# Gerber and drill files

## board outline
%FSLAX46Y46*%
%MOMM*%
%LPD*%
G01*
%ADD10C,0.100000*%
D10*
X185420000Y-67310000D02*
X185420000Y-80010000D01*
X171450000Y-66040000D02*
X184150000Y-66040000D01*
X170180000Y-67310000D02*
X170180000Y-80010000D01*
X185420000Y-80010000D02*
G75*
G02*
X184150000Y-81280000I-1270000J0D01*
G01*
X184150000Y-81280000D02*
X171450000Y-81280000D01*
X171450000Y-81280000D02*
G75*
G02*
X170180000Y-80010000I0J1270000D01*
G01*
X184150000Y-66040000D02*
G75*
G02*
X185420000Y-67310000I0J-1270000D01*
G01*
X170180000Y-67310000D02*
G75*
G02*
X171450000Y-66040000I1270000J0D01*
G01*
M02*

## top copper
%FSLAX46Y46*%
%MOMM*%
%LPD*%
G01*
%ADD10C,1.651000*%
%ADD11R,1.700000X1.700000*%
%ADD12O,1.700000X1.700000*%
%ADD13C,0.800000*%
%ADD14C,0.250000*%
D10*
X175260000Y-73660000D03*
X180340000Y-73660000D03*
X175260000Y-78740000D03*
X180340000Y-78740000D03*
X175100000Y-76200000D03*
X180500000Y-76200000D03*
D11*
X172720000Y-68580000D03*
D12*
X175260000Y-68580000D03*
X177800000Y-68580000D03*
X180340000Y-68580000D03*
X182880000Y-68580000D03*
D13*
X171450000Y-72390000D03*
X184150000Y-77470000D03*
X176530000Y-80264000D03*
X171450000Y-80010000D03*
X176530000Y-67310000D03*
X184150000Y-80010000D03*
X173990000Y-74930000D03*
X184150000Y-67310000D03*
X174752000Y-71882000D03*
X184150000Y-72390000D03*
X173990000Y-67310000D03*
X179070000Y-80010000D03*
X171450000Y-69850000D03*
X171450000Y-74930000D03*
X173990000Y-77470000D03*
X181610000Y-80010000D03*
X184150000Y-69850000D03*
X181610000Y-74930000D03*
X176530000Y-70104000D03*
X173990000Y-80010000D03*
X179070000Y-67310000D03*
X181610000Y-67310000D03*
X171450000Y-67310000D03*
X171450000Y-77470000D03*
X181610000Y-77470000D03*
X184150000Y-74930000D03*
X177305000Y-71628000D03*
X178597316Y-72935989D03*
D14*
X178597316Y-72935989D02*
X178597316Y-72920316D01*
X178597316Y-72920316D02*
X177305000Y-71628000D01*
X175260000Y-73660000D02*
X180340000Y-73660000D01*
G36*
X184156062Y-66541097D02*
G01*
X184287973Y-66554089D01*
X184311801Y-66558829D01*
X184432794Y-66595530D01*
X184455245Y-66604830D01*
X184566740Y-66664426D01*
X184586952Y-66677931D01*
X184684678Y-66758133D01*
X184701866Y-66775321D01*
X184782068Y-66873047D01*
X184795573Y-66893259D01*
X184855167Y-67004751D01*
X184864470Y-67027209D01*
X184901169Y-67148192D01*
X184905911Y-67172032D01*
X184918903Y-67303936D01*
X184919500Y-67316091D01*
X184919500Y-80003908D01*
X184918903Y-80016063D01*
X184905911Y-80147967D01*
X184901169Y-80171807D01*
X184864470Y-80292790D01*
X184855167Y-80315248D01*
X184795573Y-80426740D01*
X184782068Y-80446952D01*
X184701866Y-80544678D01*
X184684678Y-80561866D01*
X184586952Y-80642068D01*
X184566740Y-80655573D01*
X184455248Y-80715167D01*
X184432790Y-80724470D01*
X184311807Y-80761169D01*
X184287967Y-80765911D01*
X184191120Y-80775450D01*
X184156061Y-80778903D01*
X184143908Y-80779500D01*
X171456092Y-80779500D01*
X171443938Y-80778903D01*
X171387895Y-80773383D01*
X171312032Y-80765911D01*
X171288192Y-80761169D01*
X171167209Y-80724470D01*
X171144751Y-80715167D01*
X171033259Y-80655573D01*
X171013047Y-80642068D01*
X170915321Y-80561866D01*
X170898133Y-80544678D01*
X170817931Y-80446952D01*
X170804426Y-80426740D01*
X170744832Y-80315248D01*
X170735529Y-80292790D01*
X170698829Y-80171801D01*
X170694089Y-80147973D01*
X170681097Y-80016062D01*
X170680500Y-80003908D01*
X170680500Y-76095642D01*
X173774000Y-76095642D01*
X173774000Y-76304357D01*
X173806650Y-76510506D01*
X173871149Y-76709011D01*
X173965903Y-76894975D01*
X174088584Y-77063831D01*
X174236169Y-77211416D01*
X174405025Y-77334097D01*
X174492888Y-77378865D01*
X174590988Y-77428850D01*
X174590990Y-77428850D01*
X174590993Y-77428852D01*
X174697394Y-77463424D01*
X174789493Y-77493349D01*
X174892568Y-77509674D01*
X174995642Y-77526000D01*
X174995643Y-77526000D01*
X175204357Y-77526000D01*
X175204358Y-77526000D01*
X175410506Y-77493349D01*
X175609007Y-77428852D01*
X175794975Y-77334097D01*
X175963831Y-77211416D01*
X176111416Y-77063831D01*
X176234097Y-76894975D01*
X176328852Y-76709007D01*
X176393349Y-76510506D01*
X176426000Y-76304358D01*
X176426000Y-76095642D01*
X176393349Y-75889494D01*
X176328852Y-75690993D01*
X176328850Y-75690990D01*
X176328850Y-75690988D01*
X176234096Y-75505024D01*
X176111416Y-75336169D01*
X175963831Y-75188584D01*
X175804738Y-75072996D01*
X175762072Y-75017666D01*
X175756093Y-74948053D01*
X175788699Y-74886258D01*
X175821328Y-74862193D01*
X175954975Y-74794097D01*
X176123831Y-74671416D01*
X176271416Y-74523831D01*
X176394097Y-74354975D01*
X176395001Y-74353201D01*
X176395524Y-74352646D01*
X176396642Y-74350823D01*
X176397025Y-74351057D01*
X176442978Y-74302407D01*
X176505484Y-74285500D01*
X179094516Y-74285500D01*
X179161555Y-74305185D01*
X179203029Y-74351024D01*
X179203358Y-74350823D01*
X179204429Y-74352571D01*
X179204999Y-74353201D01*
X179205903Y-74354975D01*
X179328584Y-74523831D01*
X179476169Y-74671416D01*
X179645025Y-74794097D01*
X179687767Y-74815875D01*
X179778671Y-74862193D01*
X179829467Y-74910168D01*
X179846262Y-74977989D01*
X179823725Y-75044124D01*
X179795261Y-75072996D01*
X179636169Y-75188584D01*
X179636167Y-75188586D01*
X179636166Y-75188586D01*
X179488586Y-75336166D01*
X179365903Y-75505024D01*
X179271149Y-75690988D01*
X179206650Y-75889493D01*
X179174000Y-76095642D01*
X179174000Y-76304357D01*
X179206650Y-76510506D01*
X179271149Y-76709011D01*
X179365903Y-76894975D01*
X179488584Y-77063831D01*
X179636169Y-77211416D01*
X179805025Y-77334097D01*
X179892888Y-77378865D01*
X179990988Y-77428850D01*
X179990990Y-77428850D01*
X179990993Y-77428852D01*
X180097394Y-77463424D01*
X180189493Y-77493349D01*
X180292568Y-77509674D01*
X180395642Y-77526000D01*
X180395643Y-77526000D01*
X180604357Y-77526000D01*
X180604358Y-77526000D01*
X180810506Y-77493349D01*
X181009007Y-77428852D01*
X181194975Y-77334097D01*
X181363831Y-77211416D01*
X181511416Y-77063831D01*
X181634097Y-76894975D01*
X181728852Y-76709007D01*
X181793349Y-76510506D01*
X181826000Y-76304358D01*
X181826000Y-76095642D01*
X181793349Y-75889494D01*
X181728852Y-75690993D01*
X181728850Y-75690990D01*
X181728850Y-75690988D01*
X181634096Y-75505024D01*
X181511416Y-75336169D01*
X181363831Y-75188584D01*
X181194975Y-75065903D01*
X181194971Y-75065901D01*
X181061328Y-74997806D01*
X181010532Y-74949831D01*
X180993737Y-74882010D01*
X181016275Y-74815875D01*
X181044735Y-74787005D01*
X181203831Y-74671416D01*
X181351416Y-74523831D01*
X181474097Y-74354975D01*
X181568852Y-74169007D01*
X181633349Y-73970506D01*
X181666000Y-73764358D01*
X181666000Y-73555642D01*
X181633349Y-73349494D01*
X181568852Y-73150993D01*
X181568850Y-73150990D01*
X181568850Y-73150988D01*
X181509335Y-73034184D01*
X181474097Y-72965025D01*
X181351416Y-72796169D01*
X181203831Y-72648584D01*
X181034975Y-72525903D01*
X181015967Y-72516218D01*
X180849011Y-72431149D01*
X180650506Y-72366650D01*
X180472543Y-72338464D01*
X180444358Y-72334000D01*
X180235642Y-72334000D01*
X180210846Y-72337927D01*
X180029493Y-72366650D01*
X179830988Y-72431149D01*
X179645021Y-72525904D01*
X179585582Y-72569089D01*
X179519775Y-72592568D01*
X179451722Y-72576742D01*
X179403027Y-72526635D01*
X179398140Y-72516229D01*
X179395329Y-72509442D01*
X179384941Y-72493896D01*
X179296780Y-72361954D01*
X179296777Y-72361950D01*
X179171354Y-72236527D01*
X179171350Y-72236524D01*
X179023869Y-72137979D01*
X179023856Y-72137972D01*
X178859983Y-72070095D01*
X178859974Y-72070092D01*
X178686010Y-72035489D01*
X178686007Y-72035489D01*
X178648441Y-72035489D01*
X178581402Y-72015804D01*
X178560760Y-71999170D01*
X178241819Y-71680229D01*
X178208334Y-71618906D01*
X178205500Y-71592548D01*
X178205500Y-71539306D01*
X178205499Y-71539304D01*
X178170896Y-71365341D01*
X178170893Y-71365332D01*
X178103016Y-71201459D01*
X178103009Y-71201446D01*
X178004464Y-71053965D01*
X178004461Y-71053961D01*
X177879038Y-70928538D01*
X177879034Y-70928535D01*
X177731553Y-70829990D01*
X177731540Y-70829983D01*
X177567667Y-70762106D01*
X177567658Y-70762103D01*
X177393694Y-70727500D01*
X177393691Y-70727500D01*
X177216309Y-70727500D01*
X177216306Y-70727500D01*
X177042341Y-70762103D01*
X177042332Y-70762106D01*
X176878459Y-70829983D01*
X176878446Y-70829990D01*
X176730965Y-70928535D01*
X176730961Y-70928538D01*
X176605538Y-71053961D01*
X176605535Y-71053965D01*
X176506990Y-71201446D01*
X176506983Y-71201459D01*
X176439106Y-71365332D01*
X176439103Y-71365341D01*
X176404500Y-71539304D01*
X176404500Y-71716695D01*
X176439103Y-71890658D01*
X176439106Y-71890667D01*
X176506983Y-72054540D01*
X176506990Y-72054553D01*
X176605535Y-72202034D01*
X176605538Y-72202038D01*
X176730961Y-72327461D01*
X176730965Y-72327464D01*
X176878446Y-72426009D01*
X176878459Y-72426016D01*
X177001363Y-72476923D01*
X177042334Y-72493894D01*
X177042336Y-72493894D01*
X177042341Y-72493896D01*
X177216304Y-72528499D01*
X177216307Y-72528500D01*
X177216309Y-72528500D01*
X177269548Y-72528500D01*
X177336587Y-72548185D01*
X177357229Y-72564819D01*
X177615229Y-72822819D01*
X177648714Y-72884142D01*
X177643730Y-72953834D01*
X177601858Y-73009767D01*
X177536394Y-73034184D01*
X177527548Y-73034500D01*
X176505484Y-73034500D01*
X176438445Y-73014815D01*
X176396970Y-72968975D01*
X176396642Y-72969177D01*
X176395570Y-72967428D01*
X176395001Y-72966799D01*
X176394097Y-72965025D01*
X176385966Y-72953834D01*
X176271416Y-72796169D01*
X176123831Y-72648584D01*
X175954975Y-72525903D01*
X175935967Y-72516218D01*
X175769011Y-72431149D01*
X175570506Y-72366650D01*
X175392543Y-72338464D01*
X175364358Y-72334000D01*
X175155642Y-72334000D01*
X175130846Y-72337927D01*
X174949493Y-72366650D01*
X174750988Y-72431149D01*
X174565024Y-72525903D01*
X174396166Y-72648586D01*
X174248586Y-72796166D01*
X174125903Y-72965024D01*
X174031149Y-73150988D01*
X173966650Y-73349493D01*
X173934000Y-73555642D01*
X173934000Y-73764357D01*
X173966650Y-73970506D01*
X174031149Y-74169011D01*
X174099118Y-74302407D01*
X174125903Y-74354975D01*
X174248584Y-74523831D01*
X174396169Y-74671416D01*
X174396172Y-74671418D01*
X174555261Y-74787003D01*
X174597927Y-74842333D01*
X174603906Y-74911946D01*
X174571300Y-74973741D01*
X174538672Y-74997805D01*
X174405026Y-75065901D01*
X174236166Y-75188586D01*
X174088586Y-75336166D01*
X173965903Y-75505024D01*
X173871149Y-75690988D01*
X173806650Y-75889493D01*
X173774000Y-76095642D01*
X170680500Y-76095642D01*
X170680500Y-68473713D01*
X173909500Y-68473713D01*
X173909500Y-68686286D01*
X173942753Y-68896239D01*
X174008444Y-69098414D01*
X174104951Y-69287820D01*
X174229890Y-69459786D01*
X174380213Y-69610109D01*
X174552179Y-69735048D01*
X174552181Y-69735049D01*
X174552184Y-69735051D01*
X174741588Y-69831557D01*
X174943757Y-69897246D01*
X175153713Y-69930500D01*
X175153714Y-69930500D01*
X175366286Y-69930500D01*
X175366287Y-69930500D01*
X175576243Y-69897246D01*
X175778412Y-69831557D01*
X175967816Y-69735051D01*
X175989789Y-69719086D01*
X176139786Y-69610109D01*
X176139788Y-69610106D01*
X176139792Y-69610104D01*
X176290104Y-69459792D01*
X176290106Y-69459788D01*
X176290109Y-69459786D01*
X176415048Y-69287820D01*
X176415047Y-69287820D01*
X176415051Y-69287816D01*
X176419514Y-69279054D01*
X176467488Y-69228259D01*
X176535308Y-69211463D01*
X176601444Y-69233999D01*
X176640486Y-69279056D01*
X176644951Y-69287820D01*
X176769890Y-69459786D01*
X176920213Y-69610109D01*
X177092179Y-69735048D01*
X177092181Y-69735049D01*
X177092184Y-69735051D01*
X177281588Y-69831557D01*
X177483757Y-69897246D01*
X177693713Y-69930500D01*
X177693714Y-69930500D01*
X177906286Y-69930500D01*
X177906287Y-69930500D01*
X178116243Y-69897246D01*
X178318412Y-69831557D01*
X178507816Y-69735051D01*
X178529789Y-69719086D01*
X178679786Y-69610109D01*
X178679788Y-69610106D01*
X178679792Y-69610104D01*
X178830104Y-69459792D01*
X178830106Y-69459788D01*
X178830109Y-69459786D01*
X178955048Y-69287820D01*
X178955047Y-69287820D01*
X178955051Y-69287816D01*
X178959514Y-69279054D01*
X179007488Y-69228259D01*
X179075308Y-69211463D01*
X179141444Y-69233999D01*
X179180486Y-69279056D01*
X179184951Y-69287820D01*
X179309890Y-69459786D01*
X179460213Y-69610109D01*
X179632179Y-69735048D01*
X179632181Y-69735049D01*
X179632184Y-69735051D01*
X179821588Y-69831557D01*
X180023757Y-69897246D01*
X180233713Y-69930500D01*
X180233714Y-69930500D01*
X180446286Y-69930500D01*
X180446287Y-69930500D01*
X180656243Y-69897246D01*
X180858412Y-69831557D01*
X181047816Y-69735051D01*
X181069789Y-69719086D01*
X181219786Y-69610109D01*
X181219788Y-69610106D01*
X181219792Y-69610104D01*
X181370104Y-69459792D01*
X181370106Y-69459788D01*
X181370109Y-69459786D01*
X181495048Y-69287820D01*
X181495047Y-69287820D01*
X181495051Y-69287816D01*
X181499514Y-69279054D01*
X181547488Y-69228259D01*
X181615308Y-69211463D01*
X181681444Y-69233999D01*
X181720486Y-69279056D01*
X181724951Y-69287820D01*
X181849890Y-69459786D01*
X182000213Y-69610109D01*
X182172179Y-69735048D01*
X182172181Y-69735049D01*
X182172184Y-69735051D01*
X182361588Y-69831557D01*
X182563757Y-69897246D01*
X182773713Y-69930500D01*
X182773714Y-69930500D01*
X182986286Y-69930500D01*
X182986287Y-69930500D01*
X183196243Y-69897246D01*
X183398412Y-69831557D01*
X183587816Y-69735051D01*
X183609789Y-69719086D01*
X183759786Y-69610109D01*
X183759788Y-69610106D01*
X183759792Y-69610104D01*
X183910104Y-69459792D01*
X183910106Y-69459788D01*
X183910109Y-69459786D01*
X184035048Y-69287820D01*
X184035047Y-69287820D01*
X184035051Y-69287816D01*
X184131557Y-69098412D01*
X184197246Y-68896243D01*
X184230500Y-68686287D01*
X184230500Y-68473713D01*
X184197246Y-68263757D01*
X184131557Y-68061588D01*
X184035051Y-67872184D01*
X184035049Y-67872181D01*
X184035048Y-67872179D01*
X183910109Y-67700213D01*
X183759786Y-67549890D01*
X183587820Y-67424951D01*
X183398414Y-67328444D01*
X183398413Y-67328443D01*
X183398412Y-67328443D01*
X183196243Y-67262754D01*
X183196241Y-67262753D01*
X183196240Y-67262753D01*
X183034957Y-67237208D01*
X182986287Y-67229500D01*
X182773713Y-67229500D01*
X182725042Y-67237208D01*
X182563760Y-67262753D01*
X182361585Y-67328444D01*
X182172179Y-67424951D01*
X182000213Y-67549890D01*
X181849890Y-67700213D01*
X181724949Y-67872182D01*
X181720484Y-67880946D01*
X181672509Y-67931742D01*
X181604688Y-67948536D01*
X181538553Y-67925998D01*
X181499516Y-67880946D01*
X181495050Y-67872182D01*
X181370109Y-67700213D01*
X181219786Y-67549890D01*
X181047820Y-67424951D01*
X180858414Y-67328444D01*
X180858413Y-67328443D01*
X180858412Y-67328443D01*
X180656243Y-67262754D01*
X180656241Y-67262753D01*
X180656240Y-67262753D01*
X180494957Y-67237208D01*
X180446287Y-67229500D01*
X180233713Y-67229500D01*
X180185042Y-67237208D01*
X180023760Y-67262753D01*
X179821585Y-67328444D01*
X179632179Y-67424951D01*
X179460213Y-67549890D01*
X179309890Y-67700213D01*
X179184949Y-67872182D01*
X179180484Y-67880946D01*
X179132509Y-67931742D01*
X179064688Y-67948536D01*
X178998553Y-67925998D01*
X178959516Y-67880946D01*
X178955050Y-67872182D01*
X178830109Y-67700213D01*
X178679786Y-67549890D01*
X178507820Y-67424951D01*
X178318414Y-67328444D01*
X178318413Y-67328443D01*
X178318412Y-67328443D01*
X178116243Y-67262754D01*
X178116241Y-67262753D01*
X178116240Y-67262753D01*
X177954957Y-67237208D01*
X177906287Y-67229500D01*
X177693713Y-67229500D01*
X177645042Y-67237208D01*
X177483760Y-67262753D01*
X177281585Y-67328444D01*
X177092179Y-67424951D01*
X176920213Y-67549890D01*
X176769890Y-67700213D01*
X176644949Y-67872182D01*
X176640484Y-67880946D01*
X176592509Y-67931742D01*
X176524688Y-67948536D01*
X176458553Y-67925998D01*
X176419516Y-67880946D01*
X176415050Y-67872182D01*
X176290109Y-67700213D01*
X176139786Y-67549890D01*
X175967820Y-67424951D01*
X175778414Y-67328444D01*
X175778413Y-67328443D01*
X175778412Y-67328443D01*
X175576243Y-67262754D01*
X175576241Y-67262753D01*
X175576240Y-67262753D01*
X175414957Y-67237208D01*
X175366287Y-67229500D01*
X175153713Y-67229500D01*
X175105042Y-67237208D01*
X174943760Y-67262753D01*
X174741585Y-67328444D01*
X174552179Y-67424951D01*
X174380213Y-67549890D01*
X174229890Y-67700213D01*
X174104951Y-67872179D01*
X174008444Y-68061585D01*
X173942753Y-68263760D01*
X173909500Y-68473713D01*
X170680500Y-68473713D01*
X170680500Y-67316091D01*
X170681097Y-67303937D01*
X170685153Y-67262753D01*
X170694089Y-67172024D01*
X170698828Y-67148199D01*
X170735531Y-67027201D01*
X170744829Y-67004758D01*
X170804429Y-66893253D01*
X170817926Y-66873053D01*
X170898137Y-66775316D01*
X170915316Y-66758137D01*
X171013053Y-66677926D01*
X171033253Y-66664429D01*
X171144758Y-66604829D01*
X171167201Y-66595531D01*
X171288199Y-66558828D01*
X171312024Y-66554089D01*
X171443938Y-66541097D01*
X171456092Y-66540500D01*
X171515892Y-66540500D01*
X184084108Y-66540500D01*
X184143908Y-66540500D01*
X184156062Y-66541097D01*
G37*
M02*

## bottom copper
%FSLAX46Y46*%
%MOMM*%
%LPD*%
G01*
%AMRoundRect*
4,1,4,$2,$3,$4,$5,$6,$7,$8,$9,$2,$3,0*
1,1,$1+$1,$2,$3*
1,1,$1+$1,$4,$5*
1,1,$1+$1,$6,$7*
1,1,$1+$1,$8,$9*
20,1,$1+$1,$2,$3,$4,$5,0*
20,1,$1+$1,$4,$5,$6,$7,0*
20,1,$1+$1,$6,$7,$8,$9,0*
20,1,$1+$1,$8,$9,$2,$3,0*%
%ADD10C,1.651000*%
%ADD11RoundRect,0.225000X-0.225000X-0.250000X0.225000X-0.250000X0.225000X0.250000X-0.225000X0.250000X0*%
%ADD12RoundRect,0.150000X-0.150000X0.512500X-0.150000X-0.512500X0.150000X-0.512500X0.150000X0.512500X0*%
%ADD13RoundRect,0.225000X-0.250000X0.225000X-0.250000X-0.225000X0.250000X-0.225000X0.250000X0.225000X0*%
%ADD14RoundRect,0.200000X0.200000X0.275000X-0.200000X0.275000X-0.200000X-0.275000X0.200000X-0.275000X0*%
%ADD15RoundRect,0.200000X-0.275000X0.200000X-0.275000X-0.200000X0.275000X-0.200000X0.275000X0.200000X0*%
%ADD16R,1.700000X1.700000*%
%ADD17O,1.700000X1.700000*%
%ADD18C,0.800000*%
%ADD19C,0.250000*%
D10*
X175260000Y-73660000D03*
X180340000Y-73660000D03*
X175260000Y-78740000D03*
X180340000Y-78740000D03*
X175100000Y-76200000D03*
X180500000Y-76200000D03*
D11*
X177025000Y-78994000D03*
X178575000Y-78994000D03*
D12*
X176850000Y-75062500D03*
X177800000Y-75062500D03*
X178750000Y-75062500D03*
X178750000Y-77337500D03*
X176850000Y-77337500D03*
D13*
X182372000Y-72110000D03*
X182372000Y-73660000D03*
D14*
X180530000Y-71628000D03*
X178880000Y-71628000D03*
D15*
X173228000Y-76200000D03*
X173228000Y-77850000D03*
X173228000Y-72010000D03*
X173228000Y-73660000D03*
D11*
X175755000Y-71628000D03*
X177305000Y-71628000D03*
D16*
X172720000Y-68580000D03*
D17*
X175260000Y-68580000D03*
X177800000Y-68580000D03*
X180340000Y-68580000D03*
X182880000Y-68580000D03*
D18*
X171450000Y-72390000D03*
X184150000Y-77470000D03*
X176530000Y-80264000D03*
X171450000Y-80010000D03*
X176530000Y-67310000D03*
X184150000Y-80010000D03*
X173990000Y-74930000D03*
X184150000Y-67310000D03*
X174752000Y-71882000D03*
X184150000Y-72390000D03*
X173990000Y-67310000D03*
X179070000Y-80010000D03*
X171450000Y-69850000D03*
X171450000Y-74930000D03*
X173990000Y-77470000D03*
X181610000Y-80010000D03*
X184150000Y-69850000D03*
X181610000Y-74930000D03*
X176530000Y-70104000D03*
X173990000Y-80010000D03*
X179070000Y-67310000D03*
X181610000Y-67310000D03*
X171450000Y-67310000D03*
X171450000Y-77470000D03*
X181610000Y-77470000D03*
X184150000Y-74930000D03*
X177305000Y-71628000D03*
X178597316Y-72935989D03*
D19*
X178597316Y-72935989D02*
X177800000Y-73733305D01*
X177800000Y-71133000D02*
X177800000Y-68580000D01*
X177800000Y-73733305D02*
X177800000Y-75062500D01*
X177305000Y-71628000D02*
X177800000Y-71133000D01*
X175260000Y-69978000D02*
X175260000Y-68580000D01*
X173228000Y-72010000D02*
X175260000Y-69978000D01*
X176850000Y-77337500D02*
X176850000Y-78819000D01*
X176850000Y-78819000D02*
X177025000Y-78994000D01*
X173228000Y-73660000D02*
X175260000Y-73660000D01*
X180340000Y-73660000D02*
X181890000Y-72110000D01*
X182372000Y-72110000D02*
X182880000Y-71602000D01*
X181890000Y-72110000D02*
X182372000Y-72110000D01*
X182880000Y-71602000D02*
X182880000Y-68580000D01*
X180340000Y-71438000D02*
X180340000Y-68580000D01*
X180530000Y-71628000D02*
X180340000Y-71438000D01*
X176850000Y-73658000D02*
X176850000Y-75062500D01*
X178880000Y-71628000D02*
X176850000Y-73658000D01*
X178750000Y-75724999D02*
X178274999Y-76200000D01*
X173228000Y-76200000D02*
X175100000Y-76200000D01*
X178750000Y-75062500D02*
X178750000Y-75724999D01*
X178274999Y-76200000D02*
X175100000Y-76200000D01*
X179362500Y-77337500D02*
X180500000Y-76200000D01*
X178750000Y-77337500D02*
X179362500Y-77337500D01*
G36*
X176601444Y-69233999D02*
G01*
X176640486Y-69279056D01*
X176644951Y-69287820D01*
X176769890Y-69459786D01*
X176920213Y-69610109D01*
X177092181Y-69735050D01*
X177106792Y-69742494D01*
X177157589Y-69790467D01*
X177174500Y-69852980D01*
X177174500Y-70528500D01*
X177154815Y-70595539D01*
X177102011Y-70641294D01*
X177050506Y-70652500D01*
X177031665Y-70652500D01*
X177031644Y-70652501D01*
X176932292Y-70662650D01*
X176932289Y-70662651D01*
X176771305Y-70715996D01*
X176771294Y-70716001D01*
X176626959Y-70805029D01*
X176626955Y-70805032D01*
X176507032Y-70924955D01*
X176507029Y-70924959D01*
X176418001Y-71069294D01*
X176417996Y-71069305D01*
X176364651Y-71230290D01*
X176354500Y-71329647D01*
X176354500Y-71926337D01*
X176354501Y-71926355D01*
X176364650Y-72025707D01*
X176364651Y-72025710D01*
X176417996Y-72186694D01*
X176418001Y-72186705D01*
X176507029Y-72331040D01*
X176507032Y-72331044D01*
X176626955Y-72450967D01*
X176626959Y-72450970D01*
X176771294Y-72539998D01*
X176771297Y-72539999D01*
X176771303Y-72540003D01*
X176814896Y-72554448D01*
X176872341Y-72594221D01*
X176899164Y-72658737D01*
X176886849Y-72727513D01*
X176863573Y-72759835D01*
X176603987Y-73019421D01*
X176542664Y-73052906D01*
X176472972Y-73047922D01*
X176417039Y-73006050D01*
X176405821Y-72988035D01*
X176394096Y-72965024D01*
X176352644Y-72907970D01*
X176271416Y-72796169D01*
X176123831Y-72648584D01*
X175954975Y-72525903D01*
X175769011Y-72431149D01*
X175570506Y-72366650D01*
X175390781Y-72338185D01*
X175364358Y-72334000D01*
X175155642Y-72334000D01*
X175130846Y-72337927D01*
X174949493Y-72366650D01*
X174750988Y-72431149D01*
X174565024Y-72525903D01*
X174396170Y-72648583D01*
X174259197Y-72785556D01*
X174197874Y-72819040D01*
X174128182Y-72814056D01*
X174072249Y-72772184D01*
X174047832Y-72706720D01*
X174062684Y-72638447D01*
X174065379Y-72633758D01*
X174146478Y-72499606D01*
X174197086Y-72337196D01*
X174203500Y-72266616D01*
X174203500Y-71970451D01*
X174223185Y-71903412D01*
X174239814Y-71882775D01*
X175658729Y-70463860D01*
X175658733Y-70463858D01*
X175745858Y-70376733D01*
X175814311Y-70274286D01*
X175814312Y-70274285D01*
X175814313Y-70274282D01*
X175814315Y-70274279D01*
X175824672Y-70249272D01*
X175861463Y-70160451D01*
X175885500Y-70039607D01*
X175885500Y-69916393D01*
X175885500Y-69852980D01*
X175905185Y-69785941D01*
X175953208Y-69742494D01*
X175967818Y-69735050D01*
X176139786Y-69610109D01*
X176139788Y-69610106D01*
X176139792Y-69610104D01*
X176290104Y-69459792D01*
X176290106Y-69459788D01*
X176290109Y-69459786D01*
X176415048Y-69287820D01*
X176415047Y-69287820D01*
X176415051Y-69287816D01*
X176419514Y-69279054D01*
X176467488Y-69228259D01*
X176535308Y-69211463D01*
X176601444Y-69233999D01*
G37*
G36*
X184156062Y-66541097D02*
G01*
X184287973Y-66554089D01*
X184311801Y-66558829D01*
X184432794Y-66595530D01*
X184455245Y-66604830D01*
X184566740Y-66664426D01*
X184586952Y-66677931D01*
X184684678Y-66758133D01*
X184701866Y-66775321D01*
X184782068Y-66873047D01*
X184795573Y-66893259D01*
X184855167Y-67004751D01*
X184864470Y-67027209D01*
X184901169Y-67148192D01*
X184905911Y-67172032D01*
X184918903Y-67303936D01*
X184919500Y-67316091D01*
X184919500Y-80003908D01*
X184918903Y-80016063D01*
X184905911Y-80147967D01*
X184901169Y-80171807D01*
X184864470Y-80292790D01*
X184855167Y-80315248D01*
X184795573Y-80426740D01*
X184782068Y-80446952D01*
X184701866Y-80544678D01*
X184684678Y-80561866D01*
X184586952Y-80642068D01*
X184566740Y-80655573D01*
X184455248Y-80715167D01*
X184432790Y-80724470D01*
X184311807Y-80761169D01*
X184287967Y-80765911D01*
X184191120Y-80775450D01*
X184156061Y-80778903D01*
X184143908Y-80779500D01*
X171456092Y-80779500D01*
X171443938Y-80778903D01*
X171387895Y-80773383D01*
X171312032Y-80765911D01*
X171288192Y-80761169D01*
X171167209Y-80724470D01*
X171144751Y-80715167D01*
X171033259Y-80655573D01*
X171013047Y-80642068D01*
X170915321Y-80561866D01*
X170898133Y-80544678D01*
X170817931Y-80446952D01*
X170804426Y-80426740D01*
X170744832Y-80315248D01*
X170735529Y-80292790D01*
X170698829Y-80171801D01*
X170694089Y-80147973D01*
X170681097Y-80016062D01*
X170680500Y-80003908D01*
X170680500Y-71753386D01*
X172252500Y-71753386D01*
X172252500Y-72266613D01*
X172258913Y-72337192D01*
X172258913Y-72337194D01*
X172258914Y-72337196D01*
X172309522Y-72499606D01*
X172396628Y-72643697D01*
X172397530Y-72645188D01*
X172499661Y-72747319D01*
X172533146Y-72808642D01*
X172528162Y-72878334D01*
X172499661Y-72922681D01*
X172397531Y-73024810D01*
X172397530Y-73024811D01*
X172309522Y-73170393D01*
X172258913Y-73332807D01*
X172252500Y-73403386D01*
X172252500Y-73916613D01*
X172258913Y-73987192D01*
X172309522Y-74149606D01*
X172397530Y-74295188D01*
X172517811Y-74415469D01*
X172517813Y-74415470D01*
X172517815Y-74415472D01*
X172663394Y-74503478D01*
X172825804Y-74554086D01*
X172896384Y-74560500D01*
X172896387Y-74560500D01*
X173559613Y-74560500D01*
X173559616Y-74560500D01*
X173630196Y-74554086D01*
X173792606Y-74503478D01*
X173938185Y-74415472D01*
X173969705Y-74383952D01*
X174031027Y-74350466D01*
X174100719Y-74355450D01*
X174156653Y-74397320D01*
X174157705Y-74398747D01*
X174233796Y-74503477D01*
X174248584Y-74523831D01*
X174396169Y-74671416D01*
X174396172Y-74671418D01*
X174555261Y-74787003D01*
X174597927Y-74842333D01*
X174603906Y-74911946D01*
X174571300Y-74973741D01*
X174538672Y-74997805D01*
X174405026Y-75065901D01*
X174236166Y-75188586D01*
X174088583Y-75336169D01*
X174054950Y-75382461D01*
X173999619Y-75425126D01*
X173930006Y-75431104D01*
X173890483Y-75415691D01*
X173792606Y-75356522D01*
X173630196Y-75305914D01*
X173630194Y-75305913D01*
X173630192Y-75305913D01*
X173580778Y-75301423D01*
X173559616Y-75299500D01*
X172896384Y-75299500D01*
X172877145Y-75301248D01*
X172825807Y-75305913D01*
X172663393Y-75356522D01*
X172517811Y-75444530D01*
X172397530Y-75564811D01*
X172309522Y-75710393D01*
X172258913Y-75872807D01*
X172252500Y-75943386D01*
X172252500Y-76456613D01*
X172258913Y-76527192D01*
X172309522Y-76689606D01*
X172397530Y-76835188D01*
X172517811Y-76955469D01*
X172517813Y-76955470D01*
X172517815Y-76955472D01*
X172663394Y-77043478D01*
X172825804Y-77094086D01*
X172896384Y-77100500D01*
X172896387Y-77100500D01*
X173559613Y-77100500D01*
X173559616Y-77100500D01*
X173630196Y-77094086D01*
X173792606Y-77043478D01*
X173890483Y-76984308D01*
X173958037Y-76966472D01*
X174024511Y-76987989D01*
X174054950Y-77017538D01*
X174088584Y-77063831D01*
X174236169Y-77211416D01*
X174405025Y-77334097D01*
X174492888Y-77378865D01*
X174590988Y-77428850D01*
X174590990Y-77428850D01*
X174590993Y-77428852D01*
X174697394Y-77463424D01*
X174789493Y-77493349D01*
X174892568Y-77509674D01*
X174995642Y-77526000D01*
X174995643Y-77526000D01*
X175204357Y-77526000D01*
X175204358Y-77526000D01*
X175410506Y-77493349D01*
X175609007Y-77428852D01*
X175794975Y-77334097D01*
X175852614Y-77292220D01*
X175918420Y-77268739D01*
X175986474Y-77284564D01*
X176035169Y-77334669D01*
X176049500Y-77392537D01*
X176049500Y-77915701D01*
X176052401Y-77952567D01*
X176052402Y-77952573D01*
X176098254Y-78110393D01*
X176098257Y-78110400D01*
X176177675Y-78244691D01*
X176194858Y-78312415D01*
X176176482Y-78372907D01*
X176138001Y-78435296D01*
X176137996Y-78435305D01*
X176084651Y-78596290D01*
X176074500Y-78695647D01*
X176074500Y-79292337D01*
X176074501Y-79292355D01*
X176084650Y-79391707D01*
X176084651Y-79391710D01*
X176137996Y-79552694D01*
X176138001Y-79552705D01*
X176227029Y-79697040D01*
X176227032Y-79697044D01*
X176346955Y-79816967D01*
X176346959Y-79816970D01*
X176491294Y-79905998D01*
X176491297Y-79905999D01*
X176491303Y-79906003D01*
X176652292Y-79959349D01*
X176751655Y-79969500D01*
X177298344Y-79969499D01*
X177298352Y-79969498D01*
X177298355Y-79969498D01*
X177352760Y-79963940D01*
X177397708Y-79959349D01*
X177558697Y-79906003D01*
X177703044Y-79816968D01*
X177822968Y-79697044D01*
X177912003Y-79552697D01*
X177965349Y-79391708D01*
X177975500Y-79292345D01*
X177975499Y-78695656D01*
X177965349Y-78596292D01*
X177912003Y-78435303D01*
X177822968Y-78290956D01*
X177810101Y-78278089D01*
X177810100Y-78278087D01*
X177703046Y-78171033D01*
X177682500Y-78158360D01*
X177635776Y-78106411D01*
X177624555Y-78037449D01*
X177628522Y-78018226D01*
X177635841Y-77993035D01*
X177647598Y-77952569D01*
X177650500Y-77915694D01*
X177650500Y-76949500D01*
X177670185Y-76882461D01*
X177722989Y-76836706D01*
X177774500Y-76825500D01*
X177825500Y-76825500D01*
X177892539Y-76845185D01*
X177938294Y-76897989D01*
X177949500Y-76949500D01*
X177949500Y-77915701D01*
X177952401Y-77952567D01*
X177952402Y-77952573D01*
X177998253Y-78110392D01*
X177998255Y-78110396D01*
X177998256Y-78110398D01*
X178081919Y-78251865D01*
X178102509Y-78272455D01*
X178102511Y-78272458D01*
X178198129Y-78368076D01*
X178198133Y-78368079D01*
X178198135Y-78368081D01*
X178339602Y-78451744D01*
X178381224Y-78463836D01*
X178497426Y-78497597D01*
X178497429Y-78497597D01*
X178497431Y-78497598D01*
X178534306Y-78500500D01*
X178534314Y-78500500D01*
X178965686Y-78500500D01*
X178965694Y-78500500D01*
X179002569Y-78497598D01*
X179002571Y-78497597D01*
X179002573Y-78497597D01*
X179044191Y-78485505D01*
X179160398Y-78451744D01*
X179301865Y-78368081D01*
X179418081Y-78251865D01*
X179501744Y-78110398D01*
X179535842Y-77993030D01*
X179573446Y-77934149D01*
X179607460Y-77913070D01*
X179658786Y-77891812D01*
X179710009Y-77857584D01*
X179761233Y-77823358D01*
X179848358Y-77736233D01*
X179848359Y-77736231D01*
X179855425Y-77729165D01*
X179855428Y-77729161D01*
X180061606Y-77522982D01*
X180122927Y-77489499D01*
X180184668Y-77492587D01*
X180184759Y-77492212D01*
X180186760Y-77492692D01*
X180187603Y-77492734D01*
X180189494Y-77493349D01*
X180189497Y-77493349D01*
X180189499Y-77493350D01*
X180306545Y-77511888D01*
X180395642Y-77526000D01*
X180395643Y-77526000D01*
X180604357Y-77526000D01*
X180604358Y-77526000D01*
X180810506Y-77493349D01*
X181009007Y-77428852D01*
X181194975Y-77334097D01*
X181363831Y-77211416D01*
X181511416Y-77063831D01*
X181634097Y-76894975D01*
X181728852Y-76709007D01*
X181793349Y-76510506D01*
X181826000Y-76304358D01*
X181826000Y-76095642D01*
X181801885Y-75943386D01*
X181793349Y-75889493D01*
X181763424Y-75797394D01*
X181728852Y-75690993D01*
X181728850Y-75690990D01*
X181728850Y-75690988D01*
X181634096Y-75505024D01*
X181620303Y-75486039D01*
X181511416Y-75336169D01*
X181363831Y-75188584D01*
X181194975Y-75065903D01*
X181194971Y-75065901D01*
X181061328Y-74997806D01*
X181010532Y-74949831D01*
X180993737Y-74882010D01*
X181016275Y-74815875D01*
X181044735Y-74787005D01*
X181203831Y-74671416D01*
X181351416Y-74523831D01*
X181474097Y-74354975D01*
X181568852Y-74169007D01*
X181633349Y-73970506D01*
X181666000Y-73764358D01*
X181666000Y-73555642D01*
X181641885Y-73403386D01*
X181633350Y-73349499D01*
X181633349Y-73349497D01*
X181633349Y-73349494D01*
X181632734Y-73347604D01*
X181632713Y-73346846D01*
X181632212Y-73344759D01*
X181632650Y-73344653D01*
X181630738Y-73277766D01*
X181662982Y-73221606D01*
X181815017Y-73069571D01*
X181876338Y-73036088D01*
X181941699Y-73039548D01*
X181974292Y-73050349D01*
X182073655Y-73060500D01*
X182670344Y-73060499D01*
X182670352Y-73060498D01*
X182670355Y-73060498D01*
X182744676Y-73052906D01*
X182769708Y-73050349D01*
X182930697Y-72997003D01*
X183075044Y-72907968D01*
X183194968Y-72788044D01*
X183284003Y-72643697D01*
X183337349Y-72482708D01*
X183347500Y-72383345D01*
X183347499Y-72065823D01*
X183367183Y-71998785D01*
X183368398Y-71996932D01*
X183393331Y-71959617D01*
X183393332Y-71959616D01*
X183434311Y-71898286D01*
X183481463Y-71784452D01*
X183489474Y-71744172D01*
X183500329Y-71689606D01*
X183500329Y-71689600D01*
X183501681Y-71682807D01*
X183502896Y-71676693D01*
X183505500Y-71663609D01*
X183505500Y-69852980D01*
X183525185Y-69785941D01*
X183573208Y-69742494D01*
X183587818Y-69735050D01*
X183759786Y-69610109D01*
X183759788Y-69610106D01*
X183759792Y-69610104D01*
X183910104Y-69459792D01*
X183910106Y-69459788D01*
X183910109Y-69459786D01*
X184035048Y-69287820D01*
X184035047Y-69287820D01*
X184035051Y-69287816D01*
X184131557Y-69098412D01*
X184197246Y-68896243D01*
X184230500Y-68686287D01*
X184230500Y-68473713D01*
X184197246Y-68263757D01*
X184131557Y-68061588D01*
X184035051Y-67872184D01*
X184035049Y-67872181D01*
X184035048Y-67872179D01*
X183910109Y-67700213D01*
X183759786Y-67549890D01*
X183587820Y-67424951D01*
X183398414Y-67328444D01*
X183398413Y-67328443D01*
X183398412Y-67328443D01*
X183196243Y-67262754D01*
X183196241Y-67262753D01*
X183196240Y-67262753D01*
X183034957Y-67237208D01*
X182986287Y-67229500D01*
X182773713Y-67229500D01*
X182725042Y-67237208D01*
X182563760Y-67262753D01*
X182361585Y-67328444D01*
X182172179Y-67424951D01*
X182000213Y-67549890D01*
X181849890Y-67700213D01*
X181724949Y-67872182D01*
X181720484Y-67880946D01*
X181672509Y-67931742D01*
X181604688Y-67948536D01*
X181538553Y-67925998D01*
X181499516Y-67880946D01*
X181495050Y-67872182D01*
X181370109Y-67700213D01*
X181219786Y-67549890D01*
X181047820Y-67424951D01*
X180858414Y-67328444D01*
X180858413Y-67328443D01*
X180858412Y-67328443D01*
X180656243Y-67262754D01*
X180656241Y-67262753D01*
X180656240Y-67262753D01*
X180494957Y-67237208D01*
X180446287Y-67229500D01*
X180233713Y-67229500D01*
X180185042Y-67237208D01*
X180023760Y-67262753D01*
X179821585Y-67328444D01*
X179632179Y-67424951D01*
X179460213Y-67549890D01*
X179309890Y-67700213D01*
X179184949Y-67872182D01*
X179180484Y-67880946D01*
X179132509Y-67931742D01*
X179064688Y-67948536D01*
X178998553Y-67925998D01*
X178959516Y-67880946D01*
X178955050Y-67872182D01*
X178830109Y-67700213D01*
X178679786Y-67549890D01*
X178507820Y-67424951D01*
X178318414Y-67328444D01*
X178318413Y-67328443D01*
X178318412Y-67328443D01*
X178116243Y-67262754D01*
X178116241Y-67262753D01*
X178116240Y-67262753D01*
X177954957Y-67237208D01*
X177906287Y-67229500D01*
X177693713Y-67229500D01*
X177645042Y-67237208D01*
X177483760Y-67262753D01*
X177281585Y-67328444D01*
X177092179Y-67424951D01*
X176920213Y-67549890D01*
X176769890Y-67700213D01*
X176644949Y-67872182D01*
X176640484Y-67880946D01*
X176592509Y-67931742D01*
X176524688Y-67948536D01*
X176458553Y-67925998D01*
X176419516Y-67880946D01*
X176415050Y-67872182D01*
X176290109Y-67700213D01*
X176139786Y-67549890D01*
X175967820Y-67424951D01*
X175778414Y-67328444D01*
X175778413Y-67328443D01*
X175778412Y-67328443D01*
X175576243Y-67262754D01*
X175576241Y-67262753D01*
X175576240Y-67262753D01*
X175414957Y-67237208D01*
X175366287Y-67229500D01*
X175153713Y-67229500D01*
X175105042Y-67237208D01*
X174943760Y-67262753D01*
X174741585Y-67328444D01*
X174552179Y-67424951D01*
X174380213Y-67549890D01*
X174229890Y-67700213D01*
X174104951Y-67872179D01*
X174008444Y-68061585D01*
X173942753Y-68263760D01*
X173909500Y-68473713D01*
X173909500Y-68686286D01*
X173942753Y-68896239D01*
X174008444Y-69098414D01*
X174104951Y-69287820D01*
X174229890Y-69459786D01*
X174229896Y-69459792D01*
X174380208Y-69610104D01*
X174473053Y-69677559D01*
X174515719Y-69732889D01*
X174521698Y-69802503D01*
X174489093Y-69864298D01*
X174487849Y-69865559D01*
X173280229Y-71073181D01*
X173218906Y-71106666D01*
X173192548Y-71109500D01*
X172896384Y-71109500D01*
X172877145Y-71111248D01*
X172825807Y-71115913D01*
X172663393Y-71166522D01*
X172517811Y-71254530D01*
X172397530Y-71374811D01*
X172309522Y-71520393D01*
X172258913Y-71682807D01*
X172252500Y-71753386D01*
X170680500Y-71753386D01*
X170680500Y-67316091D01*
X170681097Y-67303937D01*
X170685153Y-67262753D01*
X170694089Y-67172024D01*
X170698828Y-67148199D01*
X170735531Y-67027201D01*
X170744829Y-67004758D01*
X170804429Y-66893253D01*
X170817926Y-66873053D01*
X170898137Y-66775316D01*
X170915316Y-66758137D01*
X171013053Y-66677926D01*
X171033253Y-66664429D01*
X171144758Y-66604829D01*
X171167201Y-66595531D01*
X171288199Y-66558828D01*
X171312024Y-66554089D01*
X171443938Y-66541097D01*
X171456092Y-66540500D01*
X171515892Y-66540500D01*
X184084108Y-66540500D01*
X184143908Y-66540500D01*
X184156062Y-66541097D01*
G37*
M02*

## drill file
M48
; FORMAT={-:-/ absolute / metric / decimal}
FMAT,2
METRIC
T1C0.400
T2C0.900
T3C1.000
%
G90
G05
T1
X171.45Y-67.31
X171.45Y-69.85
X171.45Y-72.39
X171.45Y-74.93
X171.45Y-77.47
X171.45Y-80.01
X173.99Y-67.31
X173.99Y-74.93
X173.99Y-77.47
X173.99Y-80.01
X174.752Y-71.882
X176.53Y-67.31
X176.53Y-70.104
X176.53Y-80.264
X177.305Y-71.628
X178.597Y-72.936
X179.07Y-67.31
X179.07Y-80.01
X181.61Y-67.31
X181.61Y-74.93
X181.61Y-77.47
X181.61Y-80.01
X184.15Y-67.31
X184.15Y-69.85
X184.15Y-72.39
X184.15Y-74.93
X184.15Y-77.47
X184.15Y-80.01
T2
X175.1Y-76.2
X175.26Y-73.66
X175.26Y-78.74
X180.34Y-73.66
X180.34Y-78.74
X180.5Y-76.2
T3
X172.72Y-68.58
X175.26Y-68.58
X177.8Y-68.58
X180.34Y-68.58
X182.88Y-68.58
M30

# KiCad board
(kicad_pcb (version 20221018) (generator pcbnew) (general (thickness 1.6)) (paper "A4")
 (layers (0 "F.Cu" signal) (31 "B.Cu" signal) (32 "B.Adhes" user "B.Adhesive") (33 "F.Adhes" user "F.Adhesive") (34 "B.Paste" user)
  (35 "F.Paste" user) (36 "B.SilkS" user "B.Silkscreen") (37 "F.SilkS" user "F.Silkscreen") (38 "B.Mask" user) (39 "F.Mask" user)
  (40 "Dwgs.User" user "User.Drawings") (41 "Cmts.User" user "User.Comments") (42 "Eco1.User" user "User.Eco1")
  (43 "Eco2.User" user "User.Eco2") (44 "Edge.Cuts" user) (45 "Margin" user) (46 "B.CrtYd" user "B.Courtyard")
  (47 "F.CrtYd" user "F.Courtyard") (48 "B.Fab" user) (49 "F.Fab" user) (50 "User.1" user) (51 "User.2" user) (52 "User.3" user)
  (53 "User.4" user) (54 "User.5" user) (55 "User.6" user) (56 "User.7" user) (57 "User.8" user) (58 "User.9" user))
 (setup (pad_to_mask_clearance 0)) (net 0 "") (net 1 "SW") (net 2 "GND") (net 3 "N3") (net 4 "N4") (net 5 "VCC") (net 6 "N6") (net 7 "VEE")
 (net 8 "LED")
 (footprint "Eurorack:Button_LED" (layer "F.Cu") (at 177.8 76.2)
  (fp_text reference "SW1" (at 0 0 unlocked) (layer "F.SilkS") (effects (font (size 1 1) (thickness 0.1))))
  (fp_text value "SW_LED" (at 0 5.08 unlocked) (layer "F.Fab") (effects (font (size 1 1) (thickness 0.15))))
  (pad "1" thru_hole circle (at -2.54 -2.54) (size 1.651 1.651) (drill 0.9) (layers "*.Cu" "*.Mask") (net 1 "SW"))
  (pad "1" thru_hole circle (at 2.54 -2.54) (size 1.651 1.651) (drill 0.9) (layers "*.Cu" "*.Mask") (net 1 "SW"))
  (pad "2" thru_hole circle (at -2.54 2.54) (size 1.651 1.651) (drill 0.9) (layers "*.Cu" "*.Mask") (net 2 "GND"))
  (pad "2" thru_hole circle (at 2.54 2.54) (size 1.651 1.651) (drill 0.9) (layers "*.Cu" "*.Mask") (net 2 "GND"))
  (pad "3" thru_hole circle (at -2.7 0) (size 1.651 1.651) (drill 0.9) (layers "*.Cu" "*.Mask") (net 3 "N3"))
  (pad "4" thru_hole circle (at 2.7 0) (size 1.651 1.651) (drill 0.9) (layers "*.Cu" "*.Mask") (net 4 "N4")))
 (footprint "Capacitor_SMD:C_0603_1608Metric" (layer "B.Cu") (at 177.8 78.994)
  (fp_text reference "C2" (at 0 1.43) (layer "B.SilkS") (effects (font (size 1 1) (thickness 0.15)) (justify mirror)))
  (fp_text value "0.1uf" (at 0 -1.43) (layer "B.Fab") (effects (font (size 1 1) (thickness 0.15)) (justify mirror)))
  (pad "1" smd roundrect (at -0.775 0) (size 0.9 0.95) (layers "B.Cu" "B.Paste" "B.Mask") (roundrect_rratio 0.25) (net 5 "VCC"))
  (pad "2" smd roundrect (at 0.775 0) (size 0.9 0.95) (layers "B.Cu" "B.Paste" "B.Mask") (roundrect_rratio 0.25) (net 2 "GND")))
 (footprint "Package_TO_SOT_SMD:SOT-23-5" (layer "B.Cu") (at 177.8 76.2 -90)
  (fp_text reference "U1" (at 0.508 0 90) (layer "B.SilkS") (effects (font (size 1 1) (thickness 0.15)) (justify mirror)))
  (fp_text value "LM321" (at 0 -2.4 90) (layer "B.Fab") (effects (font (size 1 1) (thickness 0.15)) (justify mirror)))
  (pad "1" smd roundrect (at -1.1375 0.95 270) (size 1.325 0.6) (layers "B.Cu" "B.Paste" "B.Mask") (roundrect_rratio 0.25) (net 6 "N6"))
  (pad "2" smd roundrect (at -1.1375 0 270) (size 1.325 0.6) (layers "B.Cu" "B.Paste" "B.Mask") (roundrect_rratio 0.25) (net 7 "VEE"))
  (pad "3" smd roundrect (at -1.1375 -0.95 270) (size 1.325 0.6) (layers "B.Cu" "B.Paste" "B.Mask") (roundrect_rratio 0.25) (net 3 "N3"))
  (pad "4" smd roundrect (at 1.1375 -0.95 270) (size 1.325 0.6) (layers "B.Cu" "B.Paste" "B.Mask") (roundrect_rratio 0.25) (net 4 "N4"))
  (pad "5" smd roundrect (at 1.1375 0.95 270) (size 1.325 0.6) (layers "B.Cu" "B.Paste" "B.Mask") (roundrect_rratio 0.25) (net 5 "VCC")))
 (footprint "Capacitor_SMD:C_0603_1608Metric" (layer "B.Cu") (at 182.372 72.885 -90)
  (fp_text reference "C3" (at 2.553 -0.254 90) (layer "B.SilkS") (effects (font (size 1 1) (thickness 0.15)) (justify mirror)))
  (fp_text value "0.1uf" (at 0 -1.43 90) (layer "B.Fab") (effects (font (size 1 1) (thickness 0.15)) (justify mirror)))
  (pad "1" smd roundrect (at -0.775 0 270) (size 0.9 0.95) (layers "B.Cu" "B.Paste" "B.Mask") (roundrect_rratio 0.25) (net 1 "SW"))
  (pad "2" smd roundrect (at 0.775 0 270) (size 0.9 0.95) (layers "B.Cu" "B.Paste" "B.Mask") (roundrect_rratio 0.25) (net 2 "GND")))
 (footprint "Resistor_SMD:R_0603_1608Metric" (layer "B.Cu") (at 179.705 71.628 180)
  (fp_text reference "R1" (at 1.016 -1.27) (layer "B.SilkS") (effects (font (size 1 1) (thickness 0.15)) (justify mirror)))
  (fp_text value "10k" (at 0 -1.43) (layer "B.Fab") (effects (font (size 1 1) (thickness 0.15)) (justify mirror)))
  (pad "1" smd roundrect (at -0.825 0 180) (size 0.8 0.95) (layers "B.Cu" "B.Paste" "B.Mask") (roundrect_rratio 0.25) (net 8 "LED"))
  (pad "2" smd roundrect (at 0.825 0 180) (size 0.8 0.95) (layers "B.Cu" "B.Paste" "B.Mask") (roundrect_rratio 0.25) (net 6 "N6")))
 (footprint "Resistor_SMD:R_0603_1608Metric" (layer "B.Cu") (at 173.228 77.025 -90)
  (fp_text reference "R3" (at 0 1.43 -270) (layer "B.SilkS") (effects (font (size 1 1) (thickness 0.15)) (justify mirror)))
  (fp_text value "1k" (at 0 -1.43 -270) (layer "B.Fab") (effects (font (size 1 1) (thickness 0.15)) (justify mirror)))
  (pad "1" smd roundrect (at -0.825 0 270) (size 0.8 0.95) (layers "B.Cu" "B.Paste" "B.Mask") (roundrect_rratio 0.25) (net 3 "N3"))
  (pad "2" smd roundrect (at 0.825 0 270) (size 0.8 0.95) (layers "B.Cu" "B.Paste" "B.Mask") (roundrect_rratio 0.25) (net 2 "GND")))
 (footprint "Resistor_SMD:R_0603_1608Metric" (layer "B.Cu") (at 173.228 72.835 -90)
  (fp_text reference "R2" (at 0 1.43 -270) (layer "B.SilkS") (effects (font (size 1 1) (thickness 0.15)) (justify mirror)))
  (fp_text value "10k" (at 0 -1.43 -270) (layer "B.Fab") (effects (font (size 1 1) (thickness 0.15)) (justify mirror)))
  (pad "1" smd roundrect (at -0.825 0 270) (size 0.8 0.95) (layers "B.Cu" "B.Paste" "B.Mask") (roundrect_rratio 0.25) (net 5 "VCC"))
  (pad "2" smd roundrect (at 0.825 0 270) (size 0.8 0.95) (layers "B.Cu" "B.Paste" "B.Mask") (roundrect_rratio 0.25) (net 1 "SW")))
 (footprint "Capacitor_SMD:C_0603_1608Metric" (layer "B.Cu") (at 176.53 71.628)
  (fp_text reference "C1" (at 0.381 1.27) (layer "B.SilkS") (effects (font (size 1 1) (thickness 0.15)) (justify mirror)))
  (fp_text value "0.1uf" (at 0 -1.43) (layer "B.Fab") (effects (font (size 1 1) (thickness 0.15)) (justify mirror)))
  (pad "1" smd roundrect (at -0.775 0) (size 0.9 0.95) (layers "B.Cu" "B.Paste" "B.Mask") (roundrect_rratio 0.25) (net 2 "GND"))
  (pad "2" smd roundrect (at 0.775 0) (size 0.9 0.95) (layers "B.Cu" "B.Paste" "B.Mask") (roundrect_rratio 0.25) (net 7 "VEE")))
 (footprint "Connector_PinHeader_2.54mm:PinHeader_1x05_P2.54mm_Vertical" (layer "B.Cu") (at 172.72 68.58 -90)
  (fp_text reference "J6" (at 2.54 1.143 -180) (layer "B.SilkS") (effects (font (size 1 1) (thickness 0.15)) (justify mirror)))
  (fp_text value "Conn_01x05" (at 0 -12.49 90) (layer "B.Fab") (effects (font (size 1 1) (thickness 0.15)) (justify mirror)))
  (pad "1" thru_hole rect (at 0 0 270) (size 1.7 1.7) (drill 1) (layers "*.Cu" "*.Mask") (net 2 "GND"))
  (pad "2" thru_hole oval (at 0 -2.54 270) (size 1.7 1.7) (drill 1) (layers "*.Cu" "*.Mask") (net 5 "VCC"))
  (pad "3" thru_hole oval (at 0 -5.08 270) (size 1.7 1.7) (drill 1) (layers "*.Cu" "*.Mask") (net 7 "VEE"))
  (pad "4" thru_hole oval (at 0 -7.62 270) (size 1.7 1.7) (drill 1) (layers "*.Cu" "*.Mask") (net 8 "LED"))
  (pad "5" thru_hole oval (at 0 -10.16 270) (size 1.7 1.7) (drill 1) (layers "*.Cu" "*.Mask") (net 1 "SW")))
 (gr_line (start 185.42 67.31) (end 185.42 80.01) (stroke (width 0.1) (type default)) (layer "Edge.Cuts"))
 (gr_line (start 171.45 66.04) (end 184.15 66.04) (stroke (width 0.1) (type default)) (layer "Edge.Cuts"))
 (gr_line (start 170.18 67.31) (end 170.18 80.01) (stroke (width 0.1) (type default)) (layer "Edge.Cuts"))
 (gr_arc (start 185.42 80.01) (mid 185.048026 80.908026) (end 184.15 81.28) (stroke (width 0.1) (type default)) (layer "Edge.Cuts"))
 (gr_line (start 184.15 81.28) (end 171.45 81.28) (stroke (width 0.1) (type default)) (layer "Edge.Cuts"))
 (gr_arc (start 171.45 81.28) (mid 170.551974 80.908026) (end 170.18 80.01) (stroke (width 0.1) (type default)) (layer "Edge.Cuts"))
 (gr_arc (start 184.15 66.04) (mid 185.048026 66.411974) (end 185.42 67.31) (stroke (width 0.1) (type default)) (layer "Edge.Cuts"))
 (gr_arc (start 170.18 67.31) (mid 170.551974 66.411974) (end 171.45 66.04) (stroke (width 0.1) (type default)) (layer "Edge.Cuts"))
 (via (at 171.45 72.39) (size 0.8) (drill 0.4) (layers "F.Cu" "B.Cu") (free) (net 2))
 (via (at 184.15 77.47) (size 0.8) (drill 0.4) (layers "F.Cu" "B.Cu") (free) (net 2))
 (via (at 176.53 80.264) (size 0.8) (drill 0.4) (layers "F.Cu" "B.Cu") (free) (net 2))
 (via (at 171.45 80.01) (size 0.8) (drill 0.4) (layers "F.Cu" "B.Cu") (free) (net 2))
 (via (at 176.53 67.31) (size 0.8) (drill 0.4) (layers "F.Cu" "B.Cu") (free) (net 2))
 (via (at 184.15 80.01) (size 0.8) (drill 0.4) (layers "F.Cu" "B.Cu") (free) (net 2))
 (via (at 173.99 74.93) (size 0.8) (drill 0.4) (layers "F.Cu" "B.Cu") (free) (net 2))
 (via (at 184.15 67.31) (size 0.8) (drill 0.4) (layers "F.Cu" "B.Cu") (free) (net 2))
 (via (at 174.752 71.882) (size 0.8) (drill 0.4) (layers "F.Cu" "B.Cu") (free) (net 2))
 (via (at 184.15 72.39) (size 0.8) (drill 0.4) (layers "F.Cu" "B.Cu") (free) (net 2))
 (via (at 173.99 67.31) (size 0.8) (drill 0.4) (layers "F.Cu" "B.Cu") (free) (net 2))
 (via (at 179.07 80.01) (size 0.8) (drill 0.4) (layers "F.Cu" "B.Cu") (free) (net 2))
 (via (at 171.45 69.85) (size 0.8) (drill 0.4) (layers "F.Cu" "B.Cu") (free) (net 2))
 (via (at 171.45 74.93) (size 0.8) (drill 0.4) (layers "F.Cu" "B.Cu") (free) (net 2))
 (via (at 173.99 77.47) (size 0.8) (drill 0.4) (layers "F.Cu" "B.Cu") (free) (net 2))
 (via (at 181.61 80.01) (size 0.8) (drill 0.4) (layers "F.Cu" "B.Cu") (free) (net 2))
 (via (at 184.15 69.85) (size 0.8) (drill 0.4) (layers "F.Cu" "B.Cu") (free) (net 2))
 (via (at 181.61 74.93) (size 0.8) (drill 0.4) (layers "F.Cu" "B.Cu") (free) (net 2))
 (via (at 176.53 70.104) (size 0.8) (drill 0.4) (layers "F.Cu" "B.Cu") (free) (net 2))
 (via (at 173.99 80.01) (size 0.8) (drill 0.4) (layers "F.Cu" "B.Cu") (free) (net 2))
 (via (at 179.07 67.31) (size 0.8) (drill 0.4) (layers "F.Cu" "B.Cu") (free) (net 2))
 (via (at 181.61 67.31) (size 0.8) (drill 0.4) (layers "F.Cu" "B.Cu") (free) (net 2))
 (via (at 171.45 67.31) (size 0.8) (drill 0.4) (layers "F.Cu" "B.Cu") (free) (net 2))
 (via (at 171.45 77.47) (size 0.8) (drill 0.4) (layers "F.Cu" "B.Cu") (free) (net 2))
 (via (at 181.61 77.47) (size 0.8) (drill 0.4) (layers "F.Cu" "B.Cu") (free) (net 2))
 (via (at 184.15 74.93) (size 0.8) (drill 0.4) (layers "F.Cu" "B.Cu") (free) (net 2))
 (segment (start 178.597316 72.935989) (end 178.597316 72.920316) (width 0.25) (layer "F.Cu") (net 7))
 (segment (start 178.597316 72.920316) (end 177.305 71.628) (width 0.25) (layer "F.Cu") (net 7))
 (via (at 177.305 71.628) (size 0.8) (drill 0.4) (layers "F.Cu" "B.Cu") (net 7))
 (via (at 178.597316 72.935989) (size 0.8) (drill 0.4) (layers "F.Cu" "B.Cu") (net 7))
 (segment (start 178.597316 72.935989) (end 177.8 73.733305) (width 0.25) (layer "B.Cu") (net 7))
 (segment (start 177.8 71.133) (end 177.8 68.58) (width 0.25) (layer "B.Cu") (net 7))
 (segment (start 177.8 73.733305) (end 177.8 75.0625) (width 0.25) (layer "B.Cu") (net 7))
 (segment (start 177.305 71.628) (end 177.8 71.133) (width 0.25) (layer "B.Cu") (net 7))
 (segment (start 175.26 69.978) (end 175.26 68.58) (width 0.25) (layer "B.Cu") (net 5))
 (segment (start 173.228 72.01) (end 175.26 69.978) (width 0.25) (layer "B.Cu") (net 5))
 (segment (start 176.85 77.3375) (end 176.85 78.819) (width 0.25) (layer "B.Cu") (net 5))
 (segment (start 176.85 78.819) (end 177.025 78.994) (width 0.25) (layer "B.Cu") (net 5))
 (segment (start 175.26 73.66) (end 180.34 73.66) (width 0.25) (layer "F.Cu") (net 1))
 (segment (start 173.228 73.66) (end 175.26 73.66) (width 0.25) (layer "B.Cu") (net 1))
 (segment (start 180.34 73.66) (end 181.89 72.11) (width 0.25) (layer "B.Cu") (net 1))
 (segment (start 182.372 72.11) (end 182.88 71.602) (width 0.25) (layer "B.Cu") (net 1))
 (segment (start 181.89 72.11) (end 182.372 72.11) (width 0.25) (layer "B.Cu") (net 1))
 (segment (start 182.88 71.602) (end 182.88 68.58) (width 0.25) (layer "B.Cu") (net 1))
 (segment (start 180.34 71.438) (end 180.34 68.58) (width 0.25) (layer "B.Cu") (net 8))
 (segment (start 180.53 71.628) (end 180.34 71.438) (width 0.25) (layer "B.Cu") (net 8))
 (segment (start 176.85 73.658) (end 176.85 75.0625) (width 0.25) (layer "B.Cu") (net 6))
 (segment (start 178.88 71.628) (end 176.85 73.658) (width 0.25) (layer "B.Cu") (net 6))
 (segment (start 178.75 75.724999) (end 178.274999 76.2) (width 0.25) (layer "B.Cu") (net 3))
 (segment (start 173.228 76.2) (end 175.1 76.2) (width 0.25) (layer "B.Cu") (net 3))
 (segment (start 178.75 75.0625) (end 178.75 75.724999) (width 0.25) (layer "B.Cu") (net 3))
 (segment (start 178.274999 76.2) (end 175.1 76.2) (width 0.25) (layer "B.Cu") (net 3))
 (segment (start 179.3625 77.3375) (end 180.5 76.2) (width 0.25) (layer "B.Cu") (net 4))
 (segment (start 178.75 77.3375) (end 179.3625 77.3375) (width 0.25) (layer "B.Cu") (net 4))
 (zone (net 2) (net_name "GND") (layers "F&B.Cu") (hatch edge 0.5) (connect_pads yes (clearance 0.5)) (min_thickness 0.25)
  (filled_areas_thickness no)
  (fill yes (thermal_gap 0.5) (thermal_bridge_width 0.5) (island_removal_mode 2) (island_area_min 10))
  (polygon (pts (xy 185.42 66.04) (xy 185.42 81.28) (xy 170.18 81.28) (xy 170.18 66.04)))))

